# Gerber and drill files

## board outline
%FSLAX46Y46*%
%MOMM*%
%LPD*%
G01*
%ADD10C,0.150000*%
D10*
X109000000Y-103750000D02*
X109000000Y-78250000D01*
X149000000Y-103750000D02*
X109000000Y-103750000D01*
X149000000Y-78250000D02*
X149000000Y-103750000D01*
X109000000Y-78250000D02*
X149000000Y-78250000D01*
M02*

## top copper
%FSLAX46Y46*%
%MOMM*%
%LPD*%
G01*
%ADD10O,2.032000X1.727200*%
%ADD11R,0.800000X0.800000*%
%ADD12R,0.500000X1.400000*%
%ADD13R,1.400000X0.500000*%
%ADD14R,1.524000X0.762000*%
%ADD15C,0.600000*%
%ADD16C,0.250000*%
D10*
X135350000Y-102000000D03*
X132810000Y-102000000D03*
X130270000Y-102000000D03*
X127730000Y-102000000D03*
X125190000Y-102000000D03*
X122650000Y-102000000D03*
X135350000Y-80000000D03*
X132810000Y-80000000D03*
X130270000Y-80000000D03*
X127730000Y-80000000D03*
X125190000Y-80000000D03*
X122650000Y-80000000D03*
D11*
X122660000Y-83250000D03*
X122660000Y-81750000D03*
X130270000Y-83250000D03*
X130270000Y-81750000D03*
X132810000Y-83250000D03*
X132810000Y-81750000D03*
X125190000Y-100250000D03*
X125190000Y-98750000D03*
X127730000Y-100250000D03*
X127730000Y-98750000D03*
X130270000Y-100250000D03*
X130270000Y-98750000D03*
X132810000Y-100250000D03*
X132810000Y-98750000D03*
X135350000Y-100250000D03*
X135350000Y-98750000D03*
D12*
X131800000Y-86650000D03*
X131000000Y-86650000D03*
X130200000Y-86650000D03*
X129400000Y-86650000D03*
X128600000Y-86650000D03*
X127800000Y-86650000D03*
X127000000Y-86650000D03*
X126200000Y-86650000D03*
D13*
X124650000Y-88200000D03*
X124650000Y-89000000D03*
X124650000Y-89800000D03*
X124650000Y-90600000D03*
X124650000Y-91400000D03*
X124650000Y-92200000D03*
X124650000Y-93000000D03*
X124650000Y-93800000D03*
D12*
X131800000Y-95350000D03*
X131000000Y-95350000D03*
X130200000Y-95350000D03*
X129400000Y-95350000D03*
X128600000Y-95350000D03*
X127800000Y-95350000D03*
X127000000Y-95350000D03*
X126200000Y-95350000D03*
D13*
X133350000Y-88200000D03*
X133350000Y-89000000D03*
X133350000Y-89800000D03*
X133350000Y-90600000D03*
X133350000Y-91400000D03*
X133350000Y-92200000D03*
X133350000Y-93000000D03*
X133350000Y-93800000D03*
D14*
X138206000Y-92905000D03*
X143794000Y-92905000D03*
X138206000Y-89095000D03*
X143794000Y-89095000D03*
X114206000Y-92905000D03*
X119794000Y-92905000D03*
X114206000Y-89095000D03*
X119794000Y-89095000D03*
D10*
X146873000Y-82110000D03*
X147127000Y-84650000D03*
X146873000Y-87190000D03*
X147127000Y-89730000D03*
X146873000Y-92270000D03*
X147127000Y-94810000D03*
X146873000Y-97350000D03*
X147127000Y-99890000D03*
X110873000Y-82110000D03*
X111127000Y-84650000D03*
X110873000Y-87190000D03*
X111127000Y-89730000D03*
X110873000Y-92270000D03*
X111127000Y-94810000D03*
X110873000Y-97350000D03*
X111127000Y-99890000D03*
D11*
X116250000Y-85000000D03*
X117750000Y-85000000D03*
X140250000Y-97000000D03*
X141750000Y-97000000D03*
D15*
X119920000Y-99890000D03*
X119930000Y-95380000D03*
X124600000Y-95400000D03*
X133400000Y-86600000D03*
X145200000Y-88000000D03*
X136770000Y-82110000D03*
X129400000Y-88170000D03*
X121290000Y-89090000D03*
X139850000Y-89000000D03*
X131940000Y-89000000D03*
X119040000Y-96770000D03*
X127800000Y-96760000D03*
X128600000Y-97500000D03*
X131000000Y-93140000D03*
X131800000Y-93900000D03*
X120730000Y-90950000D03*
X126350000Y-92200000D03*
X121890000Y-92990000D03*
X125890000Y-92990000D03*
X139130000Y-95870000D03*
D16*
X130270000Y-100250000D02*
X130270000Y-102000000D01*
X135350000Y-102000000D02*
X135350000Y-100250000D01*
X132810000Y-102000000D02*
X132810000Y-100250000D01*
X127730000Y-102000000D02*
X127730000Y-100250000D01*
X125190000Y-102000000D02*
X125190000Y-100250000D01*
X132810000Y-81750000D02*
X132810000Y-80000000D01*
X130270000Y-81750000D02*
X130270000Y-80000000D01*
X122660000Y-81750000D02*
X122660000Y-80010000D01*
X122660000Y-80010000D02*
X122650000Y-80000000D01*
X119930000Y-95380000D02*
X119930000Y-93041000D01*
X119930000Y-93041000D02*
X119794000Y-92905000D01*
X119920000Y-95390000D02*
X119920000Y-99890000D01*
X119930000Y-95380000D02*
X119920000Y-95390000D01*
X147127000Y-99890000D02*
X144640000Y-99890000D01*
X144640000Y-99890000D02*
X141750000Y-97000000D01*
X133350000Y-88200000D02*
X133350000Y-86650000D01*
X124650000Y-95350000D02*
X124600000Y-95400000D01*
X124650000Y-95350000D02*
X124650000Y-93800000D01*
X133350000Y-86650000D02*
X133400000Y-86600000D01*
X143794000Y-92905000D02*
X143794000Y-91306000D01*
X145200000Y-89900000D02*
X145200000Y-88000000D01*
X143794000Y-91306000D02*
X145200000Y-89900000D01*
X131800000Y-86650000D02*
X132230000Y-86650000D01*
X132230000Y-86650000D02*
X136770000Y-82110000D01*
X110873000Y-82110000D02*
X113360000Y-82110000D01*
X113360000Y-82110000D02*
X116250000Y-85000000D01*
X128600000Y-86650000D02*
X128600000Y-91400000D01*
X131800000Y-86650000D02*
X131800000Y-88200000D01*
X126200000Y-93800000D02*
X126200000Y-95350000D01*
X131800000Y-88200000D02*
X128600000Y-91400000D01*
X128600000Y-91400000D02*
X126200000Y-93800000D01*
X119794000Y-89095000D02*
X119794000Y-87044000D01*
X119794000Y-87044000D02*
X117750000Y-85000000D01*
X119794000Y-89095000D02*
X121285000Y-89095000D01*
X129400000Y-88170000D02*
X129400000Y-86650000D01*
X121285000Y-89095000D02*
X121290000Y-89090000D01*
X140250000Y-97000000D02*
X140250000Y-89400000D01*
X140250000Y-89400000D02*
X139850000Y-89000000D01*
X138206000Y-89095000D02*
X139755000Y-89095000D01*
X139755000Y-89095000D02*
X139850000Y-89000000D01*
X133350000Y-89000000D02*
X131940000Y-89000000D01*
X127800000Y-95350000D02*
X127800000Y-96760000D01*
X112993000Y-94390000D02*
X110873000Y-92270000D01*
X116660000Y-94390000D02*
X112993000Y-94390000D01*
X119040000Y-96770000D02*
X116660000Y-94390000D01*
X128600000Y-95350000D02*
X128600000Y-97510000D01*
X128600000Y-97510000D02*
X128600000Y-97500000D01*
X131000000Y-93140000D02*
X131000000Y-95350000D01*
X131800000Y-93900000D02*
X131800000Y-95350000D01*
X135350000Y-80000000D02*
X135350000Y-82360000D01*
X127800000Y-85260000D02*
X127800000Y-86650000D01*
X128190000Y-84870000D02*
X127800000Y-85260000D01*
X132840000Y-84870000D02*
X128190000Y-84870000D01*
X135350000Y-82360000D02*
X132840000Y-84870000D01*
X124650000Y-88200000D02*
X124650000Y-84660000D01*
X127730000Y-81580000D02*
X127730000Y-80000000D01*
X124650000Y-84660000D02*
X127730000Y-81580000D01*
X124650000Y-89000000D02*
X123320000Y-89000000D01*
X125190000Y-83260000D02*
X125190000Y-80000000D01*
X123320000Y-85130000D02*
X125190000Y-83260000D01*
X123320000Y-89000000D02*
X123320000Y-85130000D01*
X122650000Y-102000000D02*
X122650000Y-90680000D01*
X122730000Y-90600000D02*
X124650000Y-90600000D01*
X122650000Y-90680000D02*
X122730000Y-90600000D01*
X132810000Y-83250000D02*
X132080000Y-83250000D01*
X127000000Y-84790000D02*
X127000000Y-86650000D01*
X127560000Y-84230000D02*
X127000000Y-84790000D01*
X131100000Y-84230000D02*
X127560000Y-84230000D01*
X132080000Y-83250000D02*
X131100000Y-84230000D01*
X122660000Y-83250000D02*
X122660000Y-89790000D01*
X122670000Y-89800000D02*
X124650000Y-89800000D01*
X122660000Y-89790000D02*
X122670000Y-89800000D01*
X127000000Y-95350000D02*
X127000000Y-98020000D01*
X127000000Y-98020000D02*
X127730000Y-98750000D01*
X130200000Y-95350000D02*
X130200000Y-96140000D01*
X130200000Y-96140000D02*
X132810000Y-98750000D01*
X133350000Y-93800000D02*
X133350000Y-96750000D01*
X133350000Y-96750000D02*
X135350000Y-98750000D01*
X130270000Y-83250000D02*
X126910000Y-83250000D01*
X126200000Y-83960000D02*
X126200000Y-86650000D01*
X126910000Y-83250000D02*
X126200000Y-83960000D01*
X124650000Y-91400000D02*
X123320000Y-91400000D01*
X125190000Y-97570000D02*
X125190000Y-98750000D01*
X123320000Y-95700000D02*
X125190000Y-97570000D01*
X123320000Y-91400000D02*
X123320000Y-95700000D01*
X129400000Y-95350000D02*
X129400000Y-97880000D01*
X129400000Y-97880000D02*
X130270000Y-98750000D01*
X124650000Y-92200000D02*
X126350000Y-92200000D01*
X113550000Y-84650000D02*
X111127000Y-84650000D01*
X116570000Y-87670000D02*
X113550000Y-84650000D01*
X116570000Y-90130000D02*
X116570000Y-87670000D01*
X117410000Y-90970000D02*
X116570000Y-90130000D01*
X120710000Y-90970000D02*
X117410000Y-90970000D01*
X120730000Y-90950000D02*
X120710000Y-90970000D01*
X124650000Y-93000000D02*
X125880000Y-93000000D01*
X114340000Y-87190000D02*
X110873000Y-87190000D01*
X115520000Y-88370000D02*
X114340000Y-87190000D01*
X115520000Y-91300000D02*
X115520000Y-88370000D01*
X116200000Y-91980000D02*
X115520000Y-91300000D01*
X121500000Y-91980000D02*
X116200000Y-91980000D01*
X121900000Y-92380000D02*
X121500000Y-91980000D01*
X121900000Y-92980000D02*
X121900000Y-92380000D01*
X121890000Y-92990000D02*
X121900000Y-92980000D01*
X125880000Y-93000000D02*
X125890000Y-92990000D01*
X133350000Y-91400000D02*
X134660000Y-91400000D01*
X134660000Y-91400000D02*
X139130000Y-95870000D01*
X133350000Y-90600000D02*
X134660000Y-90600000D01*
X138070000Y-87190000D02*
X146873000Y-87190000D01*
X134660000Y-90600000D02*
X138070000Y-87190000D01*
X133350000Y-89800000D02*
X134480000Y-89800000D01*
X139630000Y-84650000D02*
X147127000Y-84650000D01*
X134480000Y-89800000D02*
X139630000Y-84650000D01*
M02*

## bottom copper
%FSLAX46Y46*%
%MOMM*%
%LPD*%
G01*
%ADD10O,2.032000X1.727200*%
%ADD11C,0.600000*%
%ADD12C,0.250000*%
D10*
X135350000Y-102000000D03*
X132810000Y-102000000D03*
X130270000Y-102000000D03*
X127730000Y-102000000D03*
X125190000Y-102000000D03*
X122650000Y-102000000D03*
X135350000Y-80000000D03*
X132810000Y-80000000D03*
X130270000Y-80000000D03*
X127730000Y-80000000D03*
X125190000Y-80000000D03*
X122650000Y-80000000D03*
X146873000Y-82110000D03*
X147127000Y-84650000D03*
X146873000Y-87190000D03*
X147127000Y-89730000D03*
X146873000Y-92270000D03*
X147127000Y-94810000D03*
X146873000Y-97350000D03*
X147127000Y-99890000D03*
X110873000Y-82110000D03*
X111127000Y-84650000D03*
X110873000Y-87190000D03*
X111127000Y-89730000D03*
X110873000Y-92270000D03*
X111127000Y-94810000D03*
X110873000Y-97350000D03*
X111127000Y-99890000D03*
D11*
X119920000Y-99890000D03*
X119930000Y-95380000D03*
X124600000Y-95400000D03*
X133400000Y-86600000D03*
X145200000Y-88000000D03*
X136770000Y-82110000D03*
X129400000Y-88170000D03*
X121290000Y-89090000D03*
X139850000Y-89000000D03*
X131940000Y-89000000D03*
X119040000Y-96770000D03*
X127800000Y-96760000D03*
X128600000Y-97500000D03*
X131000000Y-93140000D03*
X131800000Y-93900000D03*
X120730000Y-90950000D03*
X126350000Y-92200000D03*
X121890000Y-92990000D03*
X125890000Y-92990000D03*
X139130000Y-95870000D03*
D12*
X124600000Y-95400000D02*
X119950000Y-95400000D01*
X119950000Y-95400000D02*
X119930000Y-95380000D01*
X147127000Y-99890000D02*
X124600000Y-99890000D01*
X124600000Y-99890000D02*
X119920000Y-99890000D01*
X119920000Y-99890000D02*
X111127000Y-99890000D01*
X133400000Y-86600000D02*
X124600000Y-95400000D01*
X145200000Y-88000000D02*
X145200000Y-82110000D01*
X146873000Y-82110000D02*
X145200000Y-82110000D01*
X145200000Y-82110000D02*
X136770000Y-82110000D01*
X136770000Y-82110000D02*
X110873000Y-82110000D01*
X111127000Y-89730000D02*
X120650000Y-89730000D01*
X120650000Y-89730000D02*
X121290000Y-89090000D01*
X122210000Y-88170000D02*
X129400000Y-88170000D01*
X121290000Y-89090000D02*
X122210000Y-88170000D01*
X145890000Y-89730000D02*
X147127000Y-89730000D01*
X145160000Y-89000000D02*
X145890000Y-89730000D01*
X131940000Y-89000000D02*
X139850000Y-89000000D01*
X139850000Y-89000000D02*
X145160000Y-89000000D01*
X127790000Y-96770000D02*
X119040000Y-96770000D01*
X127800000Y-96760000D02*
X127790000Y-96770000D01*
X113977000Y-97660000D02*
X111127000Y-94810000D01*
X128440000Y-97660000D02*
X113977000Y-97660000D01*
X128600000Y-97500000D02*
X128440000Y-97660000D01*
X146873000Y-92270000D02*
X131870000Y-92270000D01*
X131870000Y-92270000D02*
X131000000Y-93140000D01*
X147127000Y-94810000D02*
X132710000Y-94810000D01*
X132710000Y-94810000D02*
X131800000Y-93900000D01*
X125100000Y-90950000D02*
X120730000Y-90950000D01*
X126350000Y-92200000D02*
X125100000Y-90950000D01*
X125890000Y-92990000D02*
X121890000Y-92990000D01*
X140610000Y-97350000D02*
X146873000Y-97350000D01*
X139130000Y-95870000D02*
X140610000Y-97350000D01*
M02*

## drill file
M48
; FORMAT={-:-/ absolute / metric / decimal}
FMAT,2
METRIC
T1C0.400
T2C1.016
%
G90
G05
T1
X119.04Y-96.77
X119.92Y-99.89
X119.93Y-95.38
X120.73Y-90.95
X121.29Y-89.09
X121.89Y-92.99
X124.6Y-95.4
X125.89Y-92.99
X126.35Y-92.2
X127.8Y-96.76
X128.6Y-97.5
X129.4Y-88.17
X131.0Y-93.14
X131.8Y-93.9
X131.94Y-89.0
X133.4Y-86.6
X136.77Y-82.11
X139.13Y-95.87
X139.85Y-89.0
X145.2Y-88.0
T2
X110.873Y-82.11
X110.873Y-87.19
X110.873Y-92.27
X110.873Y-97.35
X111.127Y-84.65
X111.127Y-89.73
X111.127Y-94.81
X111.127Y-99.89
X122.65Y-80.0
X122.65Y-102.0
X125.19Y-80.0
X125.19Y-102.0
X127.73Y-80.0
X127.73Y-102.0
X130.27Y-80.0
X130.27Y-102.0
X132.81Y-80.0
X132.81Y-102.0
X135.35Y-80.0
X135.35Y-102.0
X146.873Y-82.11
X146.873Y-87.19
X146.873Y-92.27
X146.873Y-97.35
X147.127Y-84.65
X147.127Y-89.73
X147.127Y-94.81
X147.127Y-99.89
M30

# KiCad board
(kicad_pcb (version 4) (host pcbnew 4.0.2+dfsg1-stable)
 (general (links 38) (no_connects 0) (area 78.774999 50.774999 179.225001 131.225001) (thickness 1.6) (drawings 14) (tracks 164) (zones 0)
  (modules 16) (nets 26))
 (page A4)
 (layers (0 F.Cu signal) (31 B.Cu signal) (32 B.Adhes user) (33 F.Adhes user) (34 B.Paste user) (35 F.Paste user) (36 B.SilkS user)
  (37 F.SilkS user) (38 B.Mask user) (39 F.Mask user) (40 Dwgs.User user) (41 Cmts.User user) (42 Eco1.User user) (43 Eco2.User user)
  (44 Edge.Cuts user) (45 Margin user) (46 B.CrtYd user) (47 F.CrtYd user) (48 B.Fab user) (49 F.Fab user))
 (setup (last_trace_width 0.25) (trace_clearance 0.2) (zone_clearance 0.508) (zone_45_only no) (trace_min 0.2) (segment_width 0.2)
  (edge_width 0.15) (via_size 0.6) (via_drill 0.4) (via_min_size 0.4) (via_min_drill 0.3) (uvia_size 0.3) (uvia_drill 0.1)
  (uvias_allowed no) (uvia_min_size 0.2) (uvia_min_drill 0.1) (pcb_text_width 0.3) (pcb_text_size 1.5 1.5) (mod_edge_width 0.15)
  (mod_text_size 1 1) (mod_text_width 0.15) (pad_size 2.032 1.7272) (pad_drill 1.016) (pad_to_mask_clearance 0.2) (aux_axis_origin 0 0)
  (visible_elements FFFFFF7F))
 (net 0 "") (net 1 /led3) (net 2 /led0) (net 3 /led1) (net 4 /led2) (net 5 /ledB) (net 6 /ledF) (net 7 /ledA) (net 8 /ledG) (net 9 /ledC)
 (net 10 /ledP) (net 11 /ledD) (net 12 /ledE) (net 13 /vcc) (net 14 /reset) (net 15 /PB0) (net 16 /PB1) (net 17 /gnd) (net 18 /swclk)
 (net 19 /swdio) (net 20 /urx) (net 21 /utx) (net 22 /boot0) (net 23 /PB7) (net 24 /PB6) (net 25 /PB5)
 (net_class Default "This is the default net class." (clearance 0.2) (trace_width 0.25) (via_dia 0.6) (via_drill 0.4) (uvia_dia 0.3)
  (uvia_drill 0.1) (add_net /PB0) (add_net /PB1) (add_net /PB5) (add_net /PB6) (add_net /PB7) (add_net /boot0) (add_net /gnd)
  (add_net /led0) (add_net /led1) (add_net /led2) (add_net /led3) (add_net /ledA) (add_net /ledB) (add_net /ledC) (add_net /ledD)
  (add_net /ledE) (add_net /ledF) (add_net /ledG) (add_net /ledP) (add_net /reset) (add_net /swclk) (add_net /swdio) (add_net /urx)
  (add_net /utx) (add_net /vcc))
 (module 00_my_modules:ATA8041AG (layer B.Cu) (at 129 91 180)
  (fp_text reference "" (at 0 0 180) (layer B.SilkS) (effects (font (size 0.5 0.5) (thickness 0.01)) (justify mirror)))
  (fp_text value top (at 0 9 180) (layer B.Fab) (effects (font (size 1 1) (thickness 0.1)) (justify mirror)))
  (pad E thru_hole oval (at -6.35 -11 180) (size 2.032 1.7272) (drill 1.016) (layers *.Cu *.Mask B.SilkS))
  (pad D thru_hole oval (at -3.81 -11 180) (size 2.032 1.7272) (drill 1.016) (layers *.Cu *.Mask B.SilkS))
  (pad P thru_hole oval (at -1.27 -11 180) (size 2.032 1.7272) (drill 1.016) (layers *.Cu *.Mask B.SilkS))
  (pad C thru_hole oval (at 1.27 -11 180) (size 2.032 1.7272) (drill 1.016) (layers *.Cu *.Mask B.SilkS))
  (pad G thru_hole oval (at 3.81 -11 180) (size 2.032 1.7272) (drill 1.016) (layers *.Cu *.Mask B.SilkS))
  (pad 3 thru_hole oval (at 6.35 -11 180) (size 2.032 1.7272) (drill 1.016) (layers *.Cu *.Mask B.SilkS) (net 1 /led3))
  (pad 0 thru_hole oval (at -6.35 11 180) (size 2.032 1.7272) (drill 1.016) (layers *.Cu *.Mask B.SilkS) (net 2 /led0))
  (pad A thru_hole oval (at -3.81 11 180) (size 2.032 1.7272) (drill 1.016) (layers *.Cu *.Mask B.SilkS))
  (pad F thru_hole oval (at -1.27 11 180) (size 2.032 1.7272) (drill 1.016) (layers *.Cu *.Mask B.SilkS))
  (pad 1 thru_hole oval (at 1.27 11 180) (size 2.032 1.7272) (drill 1.016) (layers *.Cu *.Mask B.SilkS) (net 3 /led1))
  (pad 2 thru_hole oval (at 3.81 11 180) (size 2.032 1.7272) (drill 1.016) (layers *.Cu *.Mask B.SilkS) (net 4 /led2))
  (pad B thru_hole oval (at 6.35 11 180) (size 2.032 1.7272) (drill 1.016) (layers *.Cu *.Mask B.SilkS)))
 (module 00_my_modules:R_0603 (layer F.Cu) (at 122.66 82.5 90)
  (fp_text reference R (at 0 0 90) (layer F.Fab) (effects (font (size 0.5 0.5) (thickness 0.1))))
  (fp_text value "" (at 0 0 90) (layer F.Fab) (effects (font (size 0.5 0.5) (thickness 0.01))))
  (pad 1 smd rect (at -0.75 0 90) (size 0.8 0.8) (layers F.Cu F.Paste F.Mask) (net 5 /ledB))
  (pad 2 smd rect (at 0.75 0 90) (size 0.8 0.8) (layers F.Cu F.Paste F.Mask)))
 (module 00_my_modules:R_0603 (layer F.Cu) (at 130.27 82.5 90)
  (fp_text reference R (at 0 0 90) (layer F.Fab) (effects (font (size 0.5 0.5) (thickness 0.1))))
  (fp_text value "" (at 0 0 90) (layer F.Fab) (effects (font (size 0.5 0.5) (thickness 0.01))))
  (pad 1 smd rect (at -0.75 0 90) (size 0.8 0.8) (layers F.Cu F.Paste F.Mask) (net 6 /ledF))
  (pad 2 smd rect (at 0.75 0 90) (size 0.8 0.8) (layers F.Cu F.Paste F.Mask)))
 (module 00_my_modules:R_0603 (layer F.Cu) (at 132.81 82.5 90)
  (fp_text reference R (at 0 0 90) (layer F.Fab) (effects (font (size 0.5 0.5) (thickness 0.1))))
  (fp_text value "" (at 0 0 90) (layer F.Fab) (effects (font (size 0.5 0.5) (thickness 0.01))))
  (pad 1 smd rect (at -0.75 0 90) (size 0.8 0.8) (layers F.Cu F.Paste F.Mask) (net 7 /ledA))
  (pad 2 smd rect (at 0.75 0 90) (size 0.8 0.8) (layers F.Cu F.Paste F.Mask)))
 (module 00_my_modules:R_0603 (layer F.Cu) (at 125.19 99.5 90)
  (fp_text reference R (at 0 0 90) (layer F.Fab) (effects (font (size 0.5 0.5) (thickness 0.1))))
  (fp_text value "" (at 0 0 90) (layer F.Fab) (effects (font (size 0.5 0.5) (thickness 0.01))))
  (pad 1 smd rect (at -0.75 0 90) (size 0.8 0.8) (layers F.Cu F.Paste F.Mask))
  (pad 2 smd rect (at 0.75 0 90) (size 0.8 0.8) (layers F.Cu F.Paste F.Mask) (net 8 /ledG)))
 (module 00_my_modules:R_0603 (layer F.Cu) (at 127.73 99.5 90)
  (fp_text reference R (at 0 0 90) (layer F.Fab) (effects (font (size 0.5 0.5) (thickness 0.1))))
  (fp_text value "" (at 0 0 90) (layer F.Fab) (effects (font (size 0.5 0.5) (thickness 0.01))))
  (pad 1 smd rect (at -0.75 0 90) (size 0.8 0.8) (layers F.Cu F.Paste F.Mask))
  (pad 2 smd rect (at 0.75 0 90) (size 0.8 0.8) (layers F.Cu F.Paste F.Mask) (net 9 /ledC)))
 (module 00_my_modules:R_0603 (layer F.Cu) (at 130.27 99.5 90)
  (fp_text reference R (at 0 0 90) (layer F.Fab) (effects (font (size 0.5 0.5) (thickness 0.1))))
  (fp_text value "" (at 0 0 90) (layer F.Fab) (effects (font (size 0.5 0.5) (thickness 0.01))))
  (pad 1 smd rect (at -0.75 0 90) (size 0.8 0.8) (layers F.Cu F.Paste F.Mask))
  (pad 2 smd rect (at 0.75 0 90) (size 0.8 0.8) (layers F.Cu F.Paste F.Mask) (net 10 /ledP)))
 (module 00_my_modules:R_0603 (layer F.Cu) (at 132.81 99.5 90)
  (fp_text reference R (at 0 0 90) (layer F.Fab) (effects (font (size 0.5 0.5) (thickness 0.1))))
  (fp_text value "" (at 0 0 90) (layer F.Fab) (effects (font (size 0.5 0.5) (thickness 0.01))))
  (pad 1 smd rect (at -0.75 0 90) (size 0.8 0.8) (layers F.Cu F.Paste F.Mask))
  (pad 2 smd rect (at 0.75 0 90) (size 0.8 0.8) (layers F.Cu F.Paste F.Mask) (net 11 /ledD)))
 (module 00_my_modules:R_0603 (layer F.Cu) (at 135.35 99.5 90)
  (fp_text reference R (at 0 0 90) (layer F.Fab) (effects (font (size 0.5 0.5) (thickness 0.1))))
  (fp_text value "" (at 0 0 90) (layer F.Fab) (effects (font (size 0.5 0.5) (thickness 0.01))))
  (pad 1 smd rect (at -0.75 0 90) (size 0.8 0.8) (layers F.Cu F.Paste F.Mask))
  (pad 2 smd rect (at 0.75 0 90) (size 0.8 0.8) (layers F.Cu F.Paste F.Mask) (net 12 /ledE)))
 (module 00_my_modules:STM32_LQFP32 (layer F.Cu) (at 129 91 270)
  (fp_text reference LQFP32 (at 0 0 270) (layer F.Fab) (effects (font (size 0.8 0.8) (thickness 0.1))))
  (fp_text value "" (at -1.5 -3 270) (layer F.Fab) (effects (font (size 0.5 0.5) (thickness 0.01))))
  (pad 3.3 smd rect (at -4.35 -2.8 270) (size 1.4 0.5) (layers F.Cu F.Paste F.Mask) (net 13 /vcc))
  (pad PF0 smd rect (at -4.35 -2 270) (size 1.4 0.5) (layers F.Cu F.Paste F.Mask))
  (pad PF1 smd rect (at -4.35 -1.2 270) (size 1.4 0.5) (layers F.Cu F.Paste F.Mask))
  (pad RST smd rect (at -4.35 -0.4 270) (size 1.4 0.5) (layers F.Cu F.Paste F.Mask) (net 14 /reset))
  (pad 3.3 smd rect (at -4.35 0.4 270) (size 1.4 0.5) (layers F.Cu F.Paste F.Mask) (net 13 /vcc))
  (pad PA0 smd rect (at -4.35 1.2 270) (size 1.4 0.5) (layers F.Cu F.Paste F.Mask) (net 2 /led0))
  (pad PA1 smd rect (at -4.35 2 270) (size 1.4 0.5) (layers F.Cu F.Paste F.Mask) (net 7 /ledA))
  (pad PA2 smd rect (at -4.35 2.8 270) (size 1.4 0.5) (layers F.Cu F.Paste F.Mask) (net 6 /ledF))
  (pad PA3 smd rect (at -2.8 4.35) (size 1.4 0.5) (layers F.Cu F.Paste F.Mask) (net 3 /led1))
  (pad PA4 smd rect (at -2 4.35) (size 1.4 0.5) (layers F.Cu F.Paste F.Mask) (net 4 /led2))
  (pad PA5 smd rect (at -1.2 4.35) (size 1.4 0.5) (layers F.Cu F.Paste F.Mask) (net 5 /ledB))
  (pad PA6 smd rect (at -0.4 4.35) (size 1.4 0.5) (layers F.Cu F.Paste F.Mask) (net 1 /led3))
  (pad PA7 smd rect (at 0.4 4.35) (size 1.4 0.5) (layers F.Cu F.Paste F.Mask) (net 8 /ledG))
  (pad PB0 smd rect (at 1.2 4.35) (size 1.4 0.5) (layers F.Cu F.Paste F.Mask) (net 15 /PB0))
  (pad PB1 smd rect (at 2 4.35) (size 1.4 0.5) (layers F.Cu F.Paste F.Mask) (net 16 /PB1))
  (pad GND smd rect (at 2.8 4.35) (size 1.4 0.5) (layers F.Cu F.Paste F.Mask) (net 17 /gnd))
  (pad PA14 smd rect (at 4.35 -2.8 270) (size 1.4 0.5) (layers F.Cu F.Paste F.Mask) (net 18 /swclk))
  (pad PA13 smd rect (at 4.35 -2 270) (size 1.4 0.5) (layers F.Cu F.Paste F.Mask) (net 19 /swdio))
  (pad PA12 smd rect (at 4.35 -1.2 270) (size 1.4 0.5) (layers F.Cu F.Paste F.Mask) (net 11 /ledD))
  (pad PA11 smd rect (at 4.35 -0.4 270) (size 1.4 0.5) (layers F.Cu F.Paste F.Mask) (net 10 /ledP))
  (pad PA10 smd rect (at 4.35 0.4 270) (size 1.4 0.5) (layers F.Cu F.Paste F.Mask) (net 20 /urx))
  (pad PA9 smd rect (at 4.35 1.2 270) (size 1.4 0.5) (layers F.Cu F.Paste F.Mask) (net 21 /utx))
  (pad PA8 smd rect (at 4.35 2 270) (size 1.4 0.5) (layers F.Cu F.Paste F.Mask) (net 9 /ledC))
  (pad 3.3 smd rect (at 4.35 2.8 270) (size 1.4 0.5) (layers F.Cu F.Paste F.Mask) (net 13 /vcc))
  (pad GND smd rect (at -2.8 -4.35) (size 1.4 0.5) (layers F.Cu F.Paste F.Mask) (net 17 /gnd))
  (pad BOOT smd rect (at -2 -4.35) (size 1.4 0.5) (layers F.Cu F.Paste F.Mask) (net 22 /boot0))
  (pad PB7 smd rect (at -1.2 -4.35) (size 1.4 0.5) (layers F.Cu F.Paste F.Mask) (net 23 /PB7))
  (pad PB6 smd rect (at -0.4 -4.35) (size 1.4 0.5) (layers F.Cu F.Paste F.Mask) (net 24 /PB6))
  (pad PB5 smd rect (at 0.4 -4.35) (size 1.4 0.5) (layers F.Cu F.Paste F.Mask) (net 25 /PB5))
  (pad PB4 smd rect (at 1.2 -4.35) (size 1.4 0.5) (layers F.Cu F.Paste F.Mask))
  (pad PB3 smd rect (at 2 -4.35) (size 1.4 0.5) (layers F.Cu F.Paste F.Mask))
  (pad PA15 smd rect (at 2.8 -4.35) (size 1.4 0.5) (layers F.Cu F.Paste F.Mask) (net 12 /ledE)))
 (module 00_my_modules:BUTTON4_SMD (layer F.Cu) (at 141 91)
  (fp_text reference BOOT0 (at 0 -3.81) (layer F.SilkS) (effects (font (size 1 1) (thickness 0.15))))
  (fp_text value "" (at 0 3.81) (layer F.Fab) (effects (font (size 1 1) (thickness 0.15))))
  (pad 1 smd rect (at -2.794 1.905) (size 1.524 0.762) (layers F.Cu F.Paste F.Mask))
  (pad 2 smd rect (at 2.794 1.905) (size 1.524 0.762) (layers F.Cu F.Paste F.Mask) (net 13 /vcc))
  (pad 3 smd rect (at -2.794 -1.905) (size 1.524 0.762) (layers F.Cu F.Paste F.Mask) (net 22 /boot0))
  (pad 4 smd rect (at 2.794 -1.905) (size 1.524 0.762) (layers F.Cu F.Paste F.Mask)))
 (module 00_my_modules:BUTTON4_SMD (layer F.Cu) (at 117 91)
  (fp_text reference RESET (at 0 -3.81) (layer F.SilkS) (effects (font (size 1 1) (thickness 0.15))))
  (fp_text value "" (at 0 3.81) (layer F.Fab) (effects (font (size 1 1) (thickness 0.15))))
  (pad 1 smd rect (at -2.794 1.905) (size 1.524 0.762) (layers F.Cu F.Paste F.Mask))
  (pad 2 smd rect (at 2.794 1.905) (size 1.524 0.762) (layers F.Cu F.Paste F.Mask) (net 17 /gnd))
  (pad 3 smd rect (at -2.794 -1.905) (size 1.524 0.762) (layers F.Cu F.Paste F.Mask))
  (pad 4 smd rect (at 2.794 -1.905) (size 1.524 0.762) (layers F.Cu F.Paste F.Mask) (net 14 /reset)))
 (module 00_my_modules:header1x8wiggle (layer F.Cu) (at 147 91)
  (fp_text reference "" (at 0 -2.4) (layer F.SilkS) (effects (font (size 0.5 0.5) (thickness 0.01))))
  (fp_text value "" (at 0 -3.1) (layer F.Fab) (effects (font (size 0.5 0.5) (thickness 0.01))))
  (pad 1 thru_hole oval (at -0.127 -8.89) (size 2.032 1.7272) (drill 1.016) (layers *.Cu *.Mask F.SilkS) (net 13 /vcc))
  (pad 2 thru_hole oval (at 0.127 -6.35) (size 2.032 1.7272) (drill 1.016) (layers *.Cu *.Mask F.SilkS) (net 23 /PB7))
  (pad 3 thru_hole oval (at -0.127 -3.81) (size 2.032 1.7272) (drill 1.016) (layers *.Cu *.Mask F.SilkS) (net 24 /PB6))
  (pad 4 thru_hole oval (at 0.127 -1.27) (size 2.032 1.7272) (drill 1.016) (layers *.Cu *.Mask F.SilkS) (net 22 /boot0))
  (pad 5 thru_hole oval (at -0.127 1.27) (size 2.032 1.7272) (drill 1.016) (layers *.Cu *.Mask F.SilkS) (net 19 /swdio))
  (pad 6 thru_hole oval (at 0.127 3.81) (size 2.032 1.7272) (drill 1.016) (layers *.Cu *.Mask F.SilkS) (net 18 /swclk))
  (pad 7 thru_hole oval (at -0.127 6.35) (size 2.032 1.7272) (drill 1.016) (layers *.Cu *.Mask F.SilkS) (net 25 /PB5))
  (pad 8 thru_hole oval (at 0.127 8.89) (size 2.032 1.7272) (drill 1.016) (layers *.Cu *.Mask F.SilkS) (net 17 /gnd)))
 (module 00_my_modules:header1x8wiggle (layer F.Cu) (at 111 91)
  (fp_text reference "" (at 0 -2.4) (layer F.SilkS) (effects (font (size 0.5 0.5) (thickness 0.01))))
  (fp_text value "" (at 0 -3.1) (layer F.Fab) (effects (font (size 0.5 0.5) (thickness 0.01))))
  (pad 1 thru_hole oval (at -0.127 -8.89) (size 2.032 1.7272) (drill 1.016) (layers *.Cu *.Mask F.SilkS) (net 13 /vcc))
  (pad 2 thru_hole oval (at 0.127 -6.35) (size 2.032 1.7272) (drill 1.016) (layers *.Cu *.Mask F.SilkS) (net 15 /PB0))
  (pad 3 thru_hole oval (at -0.127 -3.81) (size 2.032 1.7272) (drill 1.016) (layers *.Cu *.Mask F.SilkS) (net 16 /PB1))
  (pad 4 thru_hole oval (at 0.127 -1.27) (size 2.032 1.7272) (drill 1.016) (layers *.Cu *.Mask F.SilkS) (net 14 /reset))
  (pad 5 thru_hole oval (at -0.127 1.27) (size 2.032 1.7272) (drill 1.016) (layers *.Cu *.Mask F.SilkS) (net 21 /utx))
  (pad 6 thru_hole oval (at 0.127 3.81) (size 2.032 1.7272) (drill 1.016) (layers *.Cu *.Mask F.SilkS) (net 20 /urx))
  (pad 7 thru_hole oval (at -0.127 6.35) (size 2.032 1.7272) (drill 1.016) (layers *.Cu *.Mask F.SilkS))
  (pad 8 thru_hole oval (at 0.127 8.89) (size 2.032 1.7272) (drill 1.016) (layers *.Cu *.Mask F.SilkS) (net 17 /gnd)))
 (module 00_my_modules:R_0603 (layer F.Cu) (at 117 85)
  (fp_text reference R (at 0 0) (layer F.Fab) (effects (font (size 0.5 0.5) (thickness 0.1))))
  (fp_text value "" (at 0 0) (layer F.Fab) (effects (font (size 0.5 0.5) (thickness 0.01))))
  (pad 1 smd rect (at -0.75 0) (size 0.8 0.8) (layers F.Cu F.Paste F.Mask) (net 13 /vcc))
  (pad 2 smd rect (at 0.75 0) (size 0.8 0.8) (layers F.Cu F.Paste F.Mask) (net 14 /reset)))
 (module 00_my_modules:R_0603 (layer F.Cu) (at 141 97)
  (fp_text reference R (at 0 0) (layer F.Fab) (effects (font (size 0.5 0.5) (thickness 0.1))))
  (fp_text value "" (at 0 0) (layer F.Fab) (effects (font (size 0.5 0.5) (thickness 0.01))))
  (pad 1 smd rect (at -0.75 0) (size 0.8 0.8) (layers F.Cu F.Paste F.Mask) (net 22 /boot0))
  (pad 2 smd rect (at 0.75 0) (size 0.8 0.8) (layers F.Cu F.Paste F.Mask) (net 17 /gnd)))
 (gr_line (start 109 103.75) (end 109 78.25) (angle 90) (layer Edge.Cuts) (width 0.15))
 (gr_line (start 149 103.75) (end 109 103.75) (angle 90) (layer Edge.Cuts) (width 0.15))
 (gr_line (start 149 78.25) (end 149 103.75) (angle 90) (layer Edge.Cuts) (width 0.15))
 (gr_line (start 109 78.25) (end 149 78.25) (angle 90) (layer Edge.Cuts) (width 0.15))
 (segment (start 130.27 100.25) (end 130.27 102) (width 0.25) (layer F.Cu) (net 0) (status C00000))
 (segment (start 135.35 102) (end 135.35 100.25) (width 0.25) (layer F.Cu) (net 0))
 (segment (start 132.81 102) (end 132.81 100.25) (width 0.25) (layer F.Cu) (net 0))
 (segment (start 127.73 102) (end 127.73 100.25) (width 0.25) (layer F.Cu) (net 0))
 (segment (start 125.19 102) (end 125.19 100.25) (width 0.25) (layer F.Cu) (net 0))
 (segment (start 132.81 81.75) (end 132.81 80) (width 0.25) (layer F.Cu) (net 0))
 (segment (start 130.27 81.75) (end 130.27 80) (width 0.25) (layer F.Cu) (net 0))
 (segment (start 122.66 81.75) (end 122.66 80.01) (width 0.25) (layer F.Cu) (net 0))
 (segment (start 122.66 80.01) (end 122.65 80) (width 0.25) (layer F.Cu) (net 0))
 (segment (start 119.93 95.38) (end 119.93 93.041) (width 0.25) (layer F.Cu) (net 17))
 (segment (start 119.93 93.041) (end 119.794 92.905) (width 0.25) (layer F.Cu) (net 17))
 (segment (start 124.6 95.4) (end 119.95 95.4) (width 0.25) (layer B.Cu) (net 17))
 (via (at 119.92 99.89) (size 0.6) (drill 0.4) (layers F.Cu B.Cu) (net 17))
 (segment (start 119.92 95.39) (end 119.92 99.89) (width 0.25) (layer F.Cu) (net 17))
 (segment (start 119.93 95.38) (end 119.92 95.39) (width 0.25) (layer F.Cu) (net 17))
 (via (at 119.93 95.38) (size 0.6) (drill 0.4) (layers F.Cu B.Cu) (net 17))
 (segment (start 119.95 95.4) (end 119.93 95.38) (width 0.25) (layer B.Cu) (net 17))
 (segment (start 147.127 99.89) (end 144.64 99.89) (width 0.25) (layer F.Cu) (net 17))
 (segment (start 144.64 99.89) (end 141.75 97) (width 0.25) (layer F.Cu) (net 17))
 (segment (start 147.127 99.89) (end 124.6 99.89) (width 0.25) (layer B.Cu) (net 17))
 (segment (start 124.6 99.89) (end 119.92 99.89) (width 0.25) (layer B.Cu) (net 17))
 (segment (start 119.92 99.89) (end 111.127 99.89) (width 0.25) (layer B.Cu) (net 17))
 (segment (start 133.35 88.2) (end 133.35 86.65) (width 0.25) (layer F.Cu) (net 17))
 (segment (start 124.65 95.35) (end 124.6 95.4) (width 0.25) (layer F.Cu) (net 17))
 (via (at 124.6 95.4) (size 0.6) (drill 0.4) (layers F.Cu B.Cu) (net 17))
 (segment (start 124.65 95.35) (end 124.65 93.8) (width 0.25) (layer F.Cu) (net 17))
 (segment (start 133.4 86.6) (end 124.6 95.4) (width 0.25) (layer B.Cu) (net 17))
 (via (at 133.4 86.6) (size 0.6) (drill 0.4) (layers F.Cu B.Cu) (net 17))
 (segment (start 133.35 86.65) (end 133.4 86.6) (width 0.25) (layer F.Cu) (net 17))
 (segment (start 143.794 92.905) (end 143.794 91.306) (width 0.25) (layer F.Cu) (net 13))
 (segment (start 145.2 88) (end 145.2 82.11) (width 0.25) (layer B.Cu) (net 13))
 (via (at 145.2 88) (size 0.6) (drill 0.4) (layers F.Cu B.Cu) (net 13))
 (segment (start 145.2 89.9) (end 145.2 88) (width 0.25) (layer F.Cu) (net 13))
 (segment (start 143.794 91.306) (end 145.2 89.9) (width 0.25) (layer F.Cu) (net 13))
 (segment (start 131.8 86.65) (end 132.23 86.65) (width 0.25) (layer F.Cu) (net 13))
 (via (at 136.77 82.11) (size 0.6) (drill 0.4) (layers F.Cu B.Cu) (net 13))
 (segment (start 132.23 86.65) (end 136.77 82.11) (width 0.25) (layer F.Cu) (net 13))
 (segment (start 110.873 82.11) (end 113.36 82.11) (width 0.25) (layer F.Cu) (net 13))
 (segment (start 113.36 82.11) (end 116.25 85) (width 0.25) (layer F.Cu) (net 13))
 (segment (start 146.873 82.11) (end 145.2 82.11) (width 0.25) (layer B.Cu) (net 13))
 (segment (start 145.2 82.11) (end 136.77 82.11) (width 0.25) (layer B.Cu) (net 13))
 (segment (start 136.77 82.11) (end 110.873 82.11) (width 0.25) (layer B.Cu) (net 13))
 (segment (start 128.6 86.65) (end 128.6 91.4) (width 0.25) (layer F.Cu) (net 13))
 (segment (start 131.8 86.65) (end 131.8 88.2) (width 0.25) (layer F.Cu) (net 13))
 (segment (start 126.2 93.8) (end 126.2 95.35) (width 0.25) (layer F.Cu) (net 13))
 (segment (start 131.8 88.2) (end 128.6 91.4) (width 0.25) (layer F.Cu) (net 13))
 (segment (start 128.6 91.4) (end 126.2 93.8) (width 0.25) (layer F.Cu) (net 13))
 (segment (start 119.794 89.095) (end 119.794 87.044) (width 0.25) (layer F.Cu) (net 14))
 (segment (start 119.794 87.044) (end 117.75 85) (width 0.25) (layer F.Cu) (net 14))
 (segment (start 111.127 89.73) (end 120.65 89.73) (width 0.25) (layer B.Cu) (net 14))
 (segment (start 120.65 89.73) (end 121.29 89.09) (width 0.25) (layer B.Cu) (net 14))
 (segment (start 119.794 89.095) (end 121.285 89.095) (width 0.25) (layer F.Cu) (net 14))
 (segment (start 129.4 88.17) (end 129.4 86.65) (width 0.25) (layer F.Cu) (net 14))
 (via (at 129.4 88.17) (size 0.6) (drill 0.4) (layers F.Cu B.Cu) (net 14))
 (segment (start 122.21 88.17) (end 129.4 88.17) (width 0.25) (layer B.Cu) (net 14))
 (segment (start 121.29 89.09) (end 122.21 88.17) (width 0.25) (layer B.Cu) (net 14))
 (via (at 121.29 89.09) (size 0.6) (drill 0.4) (layers F.Cu B.Cu) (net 14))
 (segment (start 121.285 89.095) (end 121.29 89.09) (width 0.25) (layer F.Cu) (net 14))
 (segment (start 140.25 97) (end 140.25 89.4) (width 0.25) (layer F.Cu) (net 22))
 (segment (start 140.25 89.4) (end 139.85 89) (width 0.25) (layer F.Cu) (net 22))
 (via (at 139.85 89) (size 0.6) (drill 0.4) (layers F.Cu B.Cu) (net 22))
 (segment (start 138.206 89.095) (end 139.755 89.095) (width 0.25) (layer F.Cu) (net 22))
 (segment (start 139.755 89.095) (end 139.85 89) (width 0.25) (layer F.Cu) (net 22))
 (segment (start 133.35 89) (end 131.94 89) (width 0.25) (layer F.Cu) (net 22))
 (segment (start 145.89 89.73) (end 147.127 89.73) (width 0.25) (layer B.Cu) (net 22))
 (segment (start 145.16 89) (end 145.89 89.73) (width 0.25) (layer B.Cu) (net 22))
 (segment (start 131.94 89) (end 139.85 89) (width 0.25) (layer B.Cu) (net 22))
 (segment (start 139.85 89) (end 145.16 89) (width 0.25) (layer B.Cu) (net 22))
 (via (at 131.94 89) (size 0.6) (drill 0.4) (layers F.Cu B.Cu) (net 22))
 (segment (start 127.8 95.35) (end 127.8 96.76) (width 0.25) (layer F.Cu) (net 21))
 (segment (start 112.993 94.39) (end 110.873 92.27) (width 0.25) (layer F.Cu) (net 21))
 (segment (start 116.66 94.39) (end 112.993 94.39) (width 0.25) (layer F.Cu) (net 21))
 (segment (start 119.04 96.77) (end 116.66 94.39) (width 0.25) (layer F.Cu) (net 21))
 (via (at 119.04 96.77) (size 0.6) (drill 0.4) (layers F.Cu B.Cu) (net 21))
 (segment (start 127.79 96.77) (end 119.04 96.77) (width 0.25) (layer B.Cu) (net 21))
 (segment (start 127.8 96.76) (end 127.79 96.77) (width 0.25) (layer B.Cu) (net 21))
 (via (at 127.8 96.76) (size 0.6) (drill 0.4) (layers F.Cu B.Cu) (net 21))
 (segment (start 128.6 95.35) (end 128.6 97.51) (width 0.25) (layer F.Cu) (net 20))
 (segment (start 113.977 97.66) (end 111.127 94.81) (width 0.25) (layer B.Cu) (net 20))
 (segment (start 128.44 97.66) (end 113.977 97.66) (width 0.25) (layer B.Cu) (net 20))
 (segment (start 128.6 97.5) (end 128.44 97.66) (width 0.25) (layer B.Cu) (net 20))
 (via (at 128.6 97.5) (size 0.6) (drill 0.4) (layers F.Cu B.Cu) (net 20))
 (segment (start 128.6 97.51) (end 128.6 97.5) (width 0.25) (layer F.Cu) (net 20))
 (segment (start 146.873 92.27) (end 131.87 92.27) (width 0.25) (layer B.Cu) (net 19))
 (segment (start 131 93.14) (end 131 95.35) (width 0.25) (layer F.Cu) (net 19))
 (via (at 131 93.14) (size 0.6) (drill 0.4) (layers F.Cu B.Cu) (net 19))
 (segment (start 131.87 92.27) (end 131 93.14) (width 0.25) (layer B.Cu) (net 19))
 (segment (start 147.127 94.81) (end 132.71 94.81) (width 0.25) (layer B.Cu) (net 18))
 (segment (start 131.8 93.9) (end 131.8 95.35) (width 0.25) (layer F.Cu) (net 18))
 (via (at 131.8 93.9) (size 0.6) (drill 0.4) (layers F.Cu B.Cu) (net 18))
 (segment (start 132.71 94.81) (end 131.8 93.9) (width 0.25) (layer B.Cu) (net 18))
 (segment (start 135.35 80) (end 135.35 82.36) (width 0.25) (layer F.Cu) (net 2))
 (segment (start 127.8 85.26) (end 127.8 86.65) (width 0.25) (layer F.Cu) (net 2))
 (segment (start 128.19 84.87) (end 127.8 85.26) (width 0.25) (layer F.Cu) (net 2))
 (segment (start 132.84 84.87) (end 128.19 84.87) (width 0.25) (layer F.Cu) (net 2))
 (segment (start 135.35 82.36) (end 132.84 84.87) (width 0.25) (layer F.Cu) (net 2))
 (segment (start 124.65 88.2) (end 124.65 84.66) (width 0.25) (layer F.Cu) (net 3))
 (segment (start 127.73 81.58) (end 127.73 80) (width 0.25) (layer F.Cu) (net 3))
 (segment (start 124.65 84.66) (end 127.73 81.58) (width 0.25) (layer F.Cu) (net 3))
 (segment (start 124.65 89) (end 123.32 89) (width 0.25) (layer F.Cu) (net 4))
 (segment (start 125.19 83.26) (end 125.19 80) (width 0.25) (layer F.Cu) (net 4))
 (segment (start 123.32 85.13) (end 125.19 83.26) (width 0.25) (layer F.Cu) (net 4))
 (segment (start 123.32 89) (end 123.32 85.13) (width 0.25) (layer F.Cu) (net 4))
 (segment (start 122.65 102) (end 122.65 90.68) (width 0.25) (layer F.Cu) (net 1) (status 400000))
 (segment (start 122.73 90.6) (end 124.65 90.6) (width 0.25) (layer F.Cu) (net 1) (status 800000))
 (segment (start 122.65 90.68) (end 122.73 90.6) (width 0.25) (layer F.Cu) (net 1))
 (segment (start 132.81 83.25) (end 132.08 83.25) (width 0.25) (layer F.Cu) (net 7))
 (segment (start 127 84.79) (end 127 86.65) (width 0.25) (layer F.Cu) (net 7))
 (segment (start 127.56 84.23) (end 127 84.79) (width 0.25) (layer F.Cu) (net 7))
 (segment (start 131.1 84.23) (end 127.56 84.23) (width 0.25) (layer F.Cu) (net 7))
 (segment (start 132.08 83.25) (end 131.1 84.23) (width 0.25) (layer F.Cu) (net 7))
 (segment (start 122.66 83.25) (end 122.66 89.79) (width 0.25) (layer F.Cu) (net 5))
 (segment (start 122.67 89.8) (end 124.65 89.8) (width 0.25) (layer F.Cu) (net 5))
 (segment (start 122.66 89.79) (end 122.67 89.8) (width 0.25) (layer F.Cu) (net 5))
 (segment (start 127 95.35) (end 127 98.02) (width 0.25) (layer F.Cu) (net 9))
 (segment (start 127 98.02) (end 127.73 98.75) (width 0.25) (layer F.Cu) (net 9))
 (segment (start 130.2 95.35) (end 130.2 96.14) (width 0.25) (layer F.Cu) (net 11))
 (segment (start 130.2 96.14) (end 132.81 98.75) (width 0.25) (layer F.Cu) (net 11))
 (segment (start 133.35 93.8) (end 133.35 96.75) (width 0.25) (layer F.Cu) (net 12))
 (segment (start 133.35 96.75) (end 135.35 98.75) (width 0.25) (layer F.Cu) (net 12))
 (segment (start 130.27 83.25) (end 126.91 83.25) (width 0.25) (layer F.Cu) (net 6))
 (segment (start 126.2 83.96) (end 126.2 86.65) (width 0.25) (layer F.Cu) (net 6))
 (segment (start 126.91 83.25) (end 126.2 83.96) (width 0.25) (layer F.Cu) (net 6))
 (segment (start 124.65 91.4) (end 123.32 91.4) (width 0.25) (layer F.Cu) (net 8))
 (segment (start 125.19 97.57) (end 125.19 98.75) (width 0.25) (layer F.Cu) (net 8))
 (segment (start 123.32 95.7) (end 125.19 97.57) (width 0.25) (layer F.Cu) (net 8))
 (segment (start 123.32 91.4) (end 123.32 95.7) (width 0.25) (layer F.Cu) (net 8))
 (segment (start 129.4 95.35) (end 129.4 97.88) (width 0.25) (layer F.Cu) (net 10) (status 400000))
 (segment (start 129.4 97.88) (end 130.27 98.75) (width 0.25) (layer F.Cu) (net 10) (status 800000))
 (segment (start 124.65 92.2) (end 126.35 92.2) (width 0.25) (layer F.Cu) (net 15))
 (segment (start 113.55 84.65) (end 111.127 84.65) (width 0.25) (layer F.Cu) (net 15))
 (segment (start 116.57 87.67) (end 113.55 84.65) (width 0.25) (layer F.Cu) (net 15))
 (segment (start 116.57 90.13) (end 116.57 87.67) (width 0.25) (layer F.Cu) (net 15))
 (segment (start 117.41 90.97) (end 116.57 90.13) (width 0.25) (layer F.Cu) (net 15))
 (segment (start 120.71 90.97) (end 117.41 90.97) (width 0.25) (layer F.Cu) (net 15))
 (segment (start 120.73 90.95) (end 120.71 90.97) (width 0.25) (layer F.Cu) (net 15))
 (via (at 120.73 90.95) (size 0.6) (drill 0.4) (layers F.Cu B.Cu) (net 15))
 (segment (start 125.1 90.95) (end 120.73 90.95) (width 0.25) (layer B.Cu) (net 15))
 (segment (start 126.35 92.2) (end 125.1 90.95) (width 0.25) (layer B.Cu) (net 15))
 (via (at 126.35 92.2) (size 0.6) (drill 0.4) (layers F.Cu B.Cu) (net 15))
 (segment (start 124.65 93) (end 125.88 93) (width 0.25) (layer F.Cu) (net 16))
 (segment (start 114.34 87.19) (end 110.873 87.19) (width 0.25) (layer F.Cu) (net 16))
 (segment (start 115.52 88.37) (end 114.34 87.19) (width 0.25) (layer F.Cu) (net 16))
 (segment (start 115.52 91.3) (end 115.52 88.37) (width 0.25) (layer F.Cu) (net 16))
 (segment (start 116.2 91.98) (end 115.52 91.3) (width 0.25) (layer F.Cu) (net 16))
 (segment (start 121.5 91.98) (end 116.2 91.98) (width 0.25) (layer F.Cu) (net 16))
 (segment (start 121.9 92.38) (end 121.5 91.98) (width 0.25) (layer F.Cu) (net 16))
 (segment (start 121.9 92.98) (end 121.9 92.38) (width 0.25) (layer F.Cu) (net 16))
 (segment (start 121.89 92.99) (end 121.9 92.98) (width 0.25) (layer F.Cu) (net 16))
 (via (at 121.89 92.99) (size 0.6) (drill 0.4) (layers F.Cu B.Cu) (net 16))
 (segment (start 125.89 92.99) (end 121.89 92.99) (width 0.25) (layer B.Cu) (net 16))
 (via (at 125.89 92.99) (size 0.6) (drill 0.4) (layers F.Cu B.Cu) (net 16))
 (segment (start 125.88 93) (end 125.89 92.99) (width 0.25) (layer F.Cu) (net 16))
 (segment (start 133.35 91.4) (end 134.66 91.4) (width 0.25) (layer F.Cu) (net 25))
 (segment (start 140.61 97.35) (end 146.873 97.35) (width 0.25) (layer B.Cu) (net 25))
 (segment (start 139.13 95.87) (end 140.61 97.35) (width 0.25) (layer B.Cu) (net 25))
 (via (at 139.13 95.87) (size 0.6) (drill 0.4) (layers F.Cu B.Cu) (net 25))
 (segment (start 134.66 91.4) (end 139.13 95.87) (width 0.25) (layer F.Cu) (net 25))
 (segment (start 133.35 90.6) (end 134.66 90.6) (width 0.25) (layer F.Cu) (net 24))
 (segment (start 138.07 87.19) (end 146.873 87.19) (width 0.25) (layer F.Cu) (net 24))
 (segment (start 134.66 90.6) (end 138.07 87.19) (width 0.25) (layer F.Cu) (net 24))
 (segment (start 133.35 89.8) (end 134.48 89.8) (width 0.25) (layer F.Cu) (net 23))
 (segment (start 139.63 84.65) (end 147.127 84.65) (width 0.25) (layer F.Cu) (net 23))
 (segment (start 134.48 89.8) (end 139.63 84.65) (width 0.25) (layer F.Cu) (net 23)))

